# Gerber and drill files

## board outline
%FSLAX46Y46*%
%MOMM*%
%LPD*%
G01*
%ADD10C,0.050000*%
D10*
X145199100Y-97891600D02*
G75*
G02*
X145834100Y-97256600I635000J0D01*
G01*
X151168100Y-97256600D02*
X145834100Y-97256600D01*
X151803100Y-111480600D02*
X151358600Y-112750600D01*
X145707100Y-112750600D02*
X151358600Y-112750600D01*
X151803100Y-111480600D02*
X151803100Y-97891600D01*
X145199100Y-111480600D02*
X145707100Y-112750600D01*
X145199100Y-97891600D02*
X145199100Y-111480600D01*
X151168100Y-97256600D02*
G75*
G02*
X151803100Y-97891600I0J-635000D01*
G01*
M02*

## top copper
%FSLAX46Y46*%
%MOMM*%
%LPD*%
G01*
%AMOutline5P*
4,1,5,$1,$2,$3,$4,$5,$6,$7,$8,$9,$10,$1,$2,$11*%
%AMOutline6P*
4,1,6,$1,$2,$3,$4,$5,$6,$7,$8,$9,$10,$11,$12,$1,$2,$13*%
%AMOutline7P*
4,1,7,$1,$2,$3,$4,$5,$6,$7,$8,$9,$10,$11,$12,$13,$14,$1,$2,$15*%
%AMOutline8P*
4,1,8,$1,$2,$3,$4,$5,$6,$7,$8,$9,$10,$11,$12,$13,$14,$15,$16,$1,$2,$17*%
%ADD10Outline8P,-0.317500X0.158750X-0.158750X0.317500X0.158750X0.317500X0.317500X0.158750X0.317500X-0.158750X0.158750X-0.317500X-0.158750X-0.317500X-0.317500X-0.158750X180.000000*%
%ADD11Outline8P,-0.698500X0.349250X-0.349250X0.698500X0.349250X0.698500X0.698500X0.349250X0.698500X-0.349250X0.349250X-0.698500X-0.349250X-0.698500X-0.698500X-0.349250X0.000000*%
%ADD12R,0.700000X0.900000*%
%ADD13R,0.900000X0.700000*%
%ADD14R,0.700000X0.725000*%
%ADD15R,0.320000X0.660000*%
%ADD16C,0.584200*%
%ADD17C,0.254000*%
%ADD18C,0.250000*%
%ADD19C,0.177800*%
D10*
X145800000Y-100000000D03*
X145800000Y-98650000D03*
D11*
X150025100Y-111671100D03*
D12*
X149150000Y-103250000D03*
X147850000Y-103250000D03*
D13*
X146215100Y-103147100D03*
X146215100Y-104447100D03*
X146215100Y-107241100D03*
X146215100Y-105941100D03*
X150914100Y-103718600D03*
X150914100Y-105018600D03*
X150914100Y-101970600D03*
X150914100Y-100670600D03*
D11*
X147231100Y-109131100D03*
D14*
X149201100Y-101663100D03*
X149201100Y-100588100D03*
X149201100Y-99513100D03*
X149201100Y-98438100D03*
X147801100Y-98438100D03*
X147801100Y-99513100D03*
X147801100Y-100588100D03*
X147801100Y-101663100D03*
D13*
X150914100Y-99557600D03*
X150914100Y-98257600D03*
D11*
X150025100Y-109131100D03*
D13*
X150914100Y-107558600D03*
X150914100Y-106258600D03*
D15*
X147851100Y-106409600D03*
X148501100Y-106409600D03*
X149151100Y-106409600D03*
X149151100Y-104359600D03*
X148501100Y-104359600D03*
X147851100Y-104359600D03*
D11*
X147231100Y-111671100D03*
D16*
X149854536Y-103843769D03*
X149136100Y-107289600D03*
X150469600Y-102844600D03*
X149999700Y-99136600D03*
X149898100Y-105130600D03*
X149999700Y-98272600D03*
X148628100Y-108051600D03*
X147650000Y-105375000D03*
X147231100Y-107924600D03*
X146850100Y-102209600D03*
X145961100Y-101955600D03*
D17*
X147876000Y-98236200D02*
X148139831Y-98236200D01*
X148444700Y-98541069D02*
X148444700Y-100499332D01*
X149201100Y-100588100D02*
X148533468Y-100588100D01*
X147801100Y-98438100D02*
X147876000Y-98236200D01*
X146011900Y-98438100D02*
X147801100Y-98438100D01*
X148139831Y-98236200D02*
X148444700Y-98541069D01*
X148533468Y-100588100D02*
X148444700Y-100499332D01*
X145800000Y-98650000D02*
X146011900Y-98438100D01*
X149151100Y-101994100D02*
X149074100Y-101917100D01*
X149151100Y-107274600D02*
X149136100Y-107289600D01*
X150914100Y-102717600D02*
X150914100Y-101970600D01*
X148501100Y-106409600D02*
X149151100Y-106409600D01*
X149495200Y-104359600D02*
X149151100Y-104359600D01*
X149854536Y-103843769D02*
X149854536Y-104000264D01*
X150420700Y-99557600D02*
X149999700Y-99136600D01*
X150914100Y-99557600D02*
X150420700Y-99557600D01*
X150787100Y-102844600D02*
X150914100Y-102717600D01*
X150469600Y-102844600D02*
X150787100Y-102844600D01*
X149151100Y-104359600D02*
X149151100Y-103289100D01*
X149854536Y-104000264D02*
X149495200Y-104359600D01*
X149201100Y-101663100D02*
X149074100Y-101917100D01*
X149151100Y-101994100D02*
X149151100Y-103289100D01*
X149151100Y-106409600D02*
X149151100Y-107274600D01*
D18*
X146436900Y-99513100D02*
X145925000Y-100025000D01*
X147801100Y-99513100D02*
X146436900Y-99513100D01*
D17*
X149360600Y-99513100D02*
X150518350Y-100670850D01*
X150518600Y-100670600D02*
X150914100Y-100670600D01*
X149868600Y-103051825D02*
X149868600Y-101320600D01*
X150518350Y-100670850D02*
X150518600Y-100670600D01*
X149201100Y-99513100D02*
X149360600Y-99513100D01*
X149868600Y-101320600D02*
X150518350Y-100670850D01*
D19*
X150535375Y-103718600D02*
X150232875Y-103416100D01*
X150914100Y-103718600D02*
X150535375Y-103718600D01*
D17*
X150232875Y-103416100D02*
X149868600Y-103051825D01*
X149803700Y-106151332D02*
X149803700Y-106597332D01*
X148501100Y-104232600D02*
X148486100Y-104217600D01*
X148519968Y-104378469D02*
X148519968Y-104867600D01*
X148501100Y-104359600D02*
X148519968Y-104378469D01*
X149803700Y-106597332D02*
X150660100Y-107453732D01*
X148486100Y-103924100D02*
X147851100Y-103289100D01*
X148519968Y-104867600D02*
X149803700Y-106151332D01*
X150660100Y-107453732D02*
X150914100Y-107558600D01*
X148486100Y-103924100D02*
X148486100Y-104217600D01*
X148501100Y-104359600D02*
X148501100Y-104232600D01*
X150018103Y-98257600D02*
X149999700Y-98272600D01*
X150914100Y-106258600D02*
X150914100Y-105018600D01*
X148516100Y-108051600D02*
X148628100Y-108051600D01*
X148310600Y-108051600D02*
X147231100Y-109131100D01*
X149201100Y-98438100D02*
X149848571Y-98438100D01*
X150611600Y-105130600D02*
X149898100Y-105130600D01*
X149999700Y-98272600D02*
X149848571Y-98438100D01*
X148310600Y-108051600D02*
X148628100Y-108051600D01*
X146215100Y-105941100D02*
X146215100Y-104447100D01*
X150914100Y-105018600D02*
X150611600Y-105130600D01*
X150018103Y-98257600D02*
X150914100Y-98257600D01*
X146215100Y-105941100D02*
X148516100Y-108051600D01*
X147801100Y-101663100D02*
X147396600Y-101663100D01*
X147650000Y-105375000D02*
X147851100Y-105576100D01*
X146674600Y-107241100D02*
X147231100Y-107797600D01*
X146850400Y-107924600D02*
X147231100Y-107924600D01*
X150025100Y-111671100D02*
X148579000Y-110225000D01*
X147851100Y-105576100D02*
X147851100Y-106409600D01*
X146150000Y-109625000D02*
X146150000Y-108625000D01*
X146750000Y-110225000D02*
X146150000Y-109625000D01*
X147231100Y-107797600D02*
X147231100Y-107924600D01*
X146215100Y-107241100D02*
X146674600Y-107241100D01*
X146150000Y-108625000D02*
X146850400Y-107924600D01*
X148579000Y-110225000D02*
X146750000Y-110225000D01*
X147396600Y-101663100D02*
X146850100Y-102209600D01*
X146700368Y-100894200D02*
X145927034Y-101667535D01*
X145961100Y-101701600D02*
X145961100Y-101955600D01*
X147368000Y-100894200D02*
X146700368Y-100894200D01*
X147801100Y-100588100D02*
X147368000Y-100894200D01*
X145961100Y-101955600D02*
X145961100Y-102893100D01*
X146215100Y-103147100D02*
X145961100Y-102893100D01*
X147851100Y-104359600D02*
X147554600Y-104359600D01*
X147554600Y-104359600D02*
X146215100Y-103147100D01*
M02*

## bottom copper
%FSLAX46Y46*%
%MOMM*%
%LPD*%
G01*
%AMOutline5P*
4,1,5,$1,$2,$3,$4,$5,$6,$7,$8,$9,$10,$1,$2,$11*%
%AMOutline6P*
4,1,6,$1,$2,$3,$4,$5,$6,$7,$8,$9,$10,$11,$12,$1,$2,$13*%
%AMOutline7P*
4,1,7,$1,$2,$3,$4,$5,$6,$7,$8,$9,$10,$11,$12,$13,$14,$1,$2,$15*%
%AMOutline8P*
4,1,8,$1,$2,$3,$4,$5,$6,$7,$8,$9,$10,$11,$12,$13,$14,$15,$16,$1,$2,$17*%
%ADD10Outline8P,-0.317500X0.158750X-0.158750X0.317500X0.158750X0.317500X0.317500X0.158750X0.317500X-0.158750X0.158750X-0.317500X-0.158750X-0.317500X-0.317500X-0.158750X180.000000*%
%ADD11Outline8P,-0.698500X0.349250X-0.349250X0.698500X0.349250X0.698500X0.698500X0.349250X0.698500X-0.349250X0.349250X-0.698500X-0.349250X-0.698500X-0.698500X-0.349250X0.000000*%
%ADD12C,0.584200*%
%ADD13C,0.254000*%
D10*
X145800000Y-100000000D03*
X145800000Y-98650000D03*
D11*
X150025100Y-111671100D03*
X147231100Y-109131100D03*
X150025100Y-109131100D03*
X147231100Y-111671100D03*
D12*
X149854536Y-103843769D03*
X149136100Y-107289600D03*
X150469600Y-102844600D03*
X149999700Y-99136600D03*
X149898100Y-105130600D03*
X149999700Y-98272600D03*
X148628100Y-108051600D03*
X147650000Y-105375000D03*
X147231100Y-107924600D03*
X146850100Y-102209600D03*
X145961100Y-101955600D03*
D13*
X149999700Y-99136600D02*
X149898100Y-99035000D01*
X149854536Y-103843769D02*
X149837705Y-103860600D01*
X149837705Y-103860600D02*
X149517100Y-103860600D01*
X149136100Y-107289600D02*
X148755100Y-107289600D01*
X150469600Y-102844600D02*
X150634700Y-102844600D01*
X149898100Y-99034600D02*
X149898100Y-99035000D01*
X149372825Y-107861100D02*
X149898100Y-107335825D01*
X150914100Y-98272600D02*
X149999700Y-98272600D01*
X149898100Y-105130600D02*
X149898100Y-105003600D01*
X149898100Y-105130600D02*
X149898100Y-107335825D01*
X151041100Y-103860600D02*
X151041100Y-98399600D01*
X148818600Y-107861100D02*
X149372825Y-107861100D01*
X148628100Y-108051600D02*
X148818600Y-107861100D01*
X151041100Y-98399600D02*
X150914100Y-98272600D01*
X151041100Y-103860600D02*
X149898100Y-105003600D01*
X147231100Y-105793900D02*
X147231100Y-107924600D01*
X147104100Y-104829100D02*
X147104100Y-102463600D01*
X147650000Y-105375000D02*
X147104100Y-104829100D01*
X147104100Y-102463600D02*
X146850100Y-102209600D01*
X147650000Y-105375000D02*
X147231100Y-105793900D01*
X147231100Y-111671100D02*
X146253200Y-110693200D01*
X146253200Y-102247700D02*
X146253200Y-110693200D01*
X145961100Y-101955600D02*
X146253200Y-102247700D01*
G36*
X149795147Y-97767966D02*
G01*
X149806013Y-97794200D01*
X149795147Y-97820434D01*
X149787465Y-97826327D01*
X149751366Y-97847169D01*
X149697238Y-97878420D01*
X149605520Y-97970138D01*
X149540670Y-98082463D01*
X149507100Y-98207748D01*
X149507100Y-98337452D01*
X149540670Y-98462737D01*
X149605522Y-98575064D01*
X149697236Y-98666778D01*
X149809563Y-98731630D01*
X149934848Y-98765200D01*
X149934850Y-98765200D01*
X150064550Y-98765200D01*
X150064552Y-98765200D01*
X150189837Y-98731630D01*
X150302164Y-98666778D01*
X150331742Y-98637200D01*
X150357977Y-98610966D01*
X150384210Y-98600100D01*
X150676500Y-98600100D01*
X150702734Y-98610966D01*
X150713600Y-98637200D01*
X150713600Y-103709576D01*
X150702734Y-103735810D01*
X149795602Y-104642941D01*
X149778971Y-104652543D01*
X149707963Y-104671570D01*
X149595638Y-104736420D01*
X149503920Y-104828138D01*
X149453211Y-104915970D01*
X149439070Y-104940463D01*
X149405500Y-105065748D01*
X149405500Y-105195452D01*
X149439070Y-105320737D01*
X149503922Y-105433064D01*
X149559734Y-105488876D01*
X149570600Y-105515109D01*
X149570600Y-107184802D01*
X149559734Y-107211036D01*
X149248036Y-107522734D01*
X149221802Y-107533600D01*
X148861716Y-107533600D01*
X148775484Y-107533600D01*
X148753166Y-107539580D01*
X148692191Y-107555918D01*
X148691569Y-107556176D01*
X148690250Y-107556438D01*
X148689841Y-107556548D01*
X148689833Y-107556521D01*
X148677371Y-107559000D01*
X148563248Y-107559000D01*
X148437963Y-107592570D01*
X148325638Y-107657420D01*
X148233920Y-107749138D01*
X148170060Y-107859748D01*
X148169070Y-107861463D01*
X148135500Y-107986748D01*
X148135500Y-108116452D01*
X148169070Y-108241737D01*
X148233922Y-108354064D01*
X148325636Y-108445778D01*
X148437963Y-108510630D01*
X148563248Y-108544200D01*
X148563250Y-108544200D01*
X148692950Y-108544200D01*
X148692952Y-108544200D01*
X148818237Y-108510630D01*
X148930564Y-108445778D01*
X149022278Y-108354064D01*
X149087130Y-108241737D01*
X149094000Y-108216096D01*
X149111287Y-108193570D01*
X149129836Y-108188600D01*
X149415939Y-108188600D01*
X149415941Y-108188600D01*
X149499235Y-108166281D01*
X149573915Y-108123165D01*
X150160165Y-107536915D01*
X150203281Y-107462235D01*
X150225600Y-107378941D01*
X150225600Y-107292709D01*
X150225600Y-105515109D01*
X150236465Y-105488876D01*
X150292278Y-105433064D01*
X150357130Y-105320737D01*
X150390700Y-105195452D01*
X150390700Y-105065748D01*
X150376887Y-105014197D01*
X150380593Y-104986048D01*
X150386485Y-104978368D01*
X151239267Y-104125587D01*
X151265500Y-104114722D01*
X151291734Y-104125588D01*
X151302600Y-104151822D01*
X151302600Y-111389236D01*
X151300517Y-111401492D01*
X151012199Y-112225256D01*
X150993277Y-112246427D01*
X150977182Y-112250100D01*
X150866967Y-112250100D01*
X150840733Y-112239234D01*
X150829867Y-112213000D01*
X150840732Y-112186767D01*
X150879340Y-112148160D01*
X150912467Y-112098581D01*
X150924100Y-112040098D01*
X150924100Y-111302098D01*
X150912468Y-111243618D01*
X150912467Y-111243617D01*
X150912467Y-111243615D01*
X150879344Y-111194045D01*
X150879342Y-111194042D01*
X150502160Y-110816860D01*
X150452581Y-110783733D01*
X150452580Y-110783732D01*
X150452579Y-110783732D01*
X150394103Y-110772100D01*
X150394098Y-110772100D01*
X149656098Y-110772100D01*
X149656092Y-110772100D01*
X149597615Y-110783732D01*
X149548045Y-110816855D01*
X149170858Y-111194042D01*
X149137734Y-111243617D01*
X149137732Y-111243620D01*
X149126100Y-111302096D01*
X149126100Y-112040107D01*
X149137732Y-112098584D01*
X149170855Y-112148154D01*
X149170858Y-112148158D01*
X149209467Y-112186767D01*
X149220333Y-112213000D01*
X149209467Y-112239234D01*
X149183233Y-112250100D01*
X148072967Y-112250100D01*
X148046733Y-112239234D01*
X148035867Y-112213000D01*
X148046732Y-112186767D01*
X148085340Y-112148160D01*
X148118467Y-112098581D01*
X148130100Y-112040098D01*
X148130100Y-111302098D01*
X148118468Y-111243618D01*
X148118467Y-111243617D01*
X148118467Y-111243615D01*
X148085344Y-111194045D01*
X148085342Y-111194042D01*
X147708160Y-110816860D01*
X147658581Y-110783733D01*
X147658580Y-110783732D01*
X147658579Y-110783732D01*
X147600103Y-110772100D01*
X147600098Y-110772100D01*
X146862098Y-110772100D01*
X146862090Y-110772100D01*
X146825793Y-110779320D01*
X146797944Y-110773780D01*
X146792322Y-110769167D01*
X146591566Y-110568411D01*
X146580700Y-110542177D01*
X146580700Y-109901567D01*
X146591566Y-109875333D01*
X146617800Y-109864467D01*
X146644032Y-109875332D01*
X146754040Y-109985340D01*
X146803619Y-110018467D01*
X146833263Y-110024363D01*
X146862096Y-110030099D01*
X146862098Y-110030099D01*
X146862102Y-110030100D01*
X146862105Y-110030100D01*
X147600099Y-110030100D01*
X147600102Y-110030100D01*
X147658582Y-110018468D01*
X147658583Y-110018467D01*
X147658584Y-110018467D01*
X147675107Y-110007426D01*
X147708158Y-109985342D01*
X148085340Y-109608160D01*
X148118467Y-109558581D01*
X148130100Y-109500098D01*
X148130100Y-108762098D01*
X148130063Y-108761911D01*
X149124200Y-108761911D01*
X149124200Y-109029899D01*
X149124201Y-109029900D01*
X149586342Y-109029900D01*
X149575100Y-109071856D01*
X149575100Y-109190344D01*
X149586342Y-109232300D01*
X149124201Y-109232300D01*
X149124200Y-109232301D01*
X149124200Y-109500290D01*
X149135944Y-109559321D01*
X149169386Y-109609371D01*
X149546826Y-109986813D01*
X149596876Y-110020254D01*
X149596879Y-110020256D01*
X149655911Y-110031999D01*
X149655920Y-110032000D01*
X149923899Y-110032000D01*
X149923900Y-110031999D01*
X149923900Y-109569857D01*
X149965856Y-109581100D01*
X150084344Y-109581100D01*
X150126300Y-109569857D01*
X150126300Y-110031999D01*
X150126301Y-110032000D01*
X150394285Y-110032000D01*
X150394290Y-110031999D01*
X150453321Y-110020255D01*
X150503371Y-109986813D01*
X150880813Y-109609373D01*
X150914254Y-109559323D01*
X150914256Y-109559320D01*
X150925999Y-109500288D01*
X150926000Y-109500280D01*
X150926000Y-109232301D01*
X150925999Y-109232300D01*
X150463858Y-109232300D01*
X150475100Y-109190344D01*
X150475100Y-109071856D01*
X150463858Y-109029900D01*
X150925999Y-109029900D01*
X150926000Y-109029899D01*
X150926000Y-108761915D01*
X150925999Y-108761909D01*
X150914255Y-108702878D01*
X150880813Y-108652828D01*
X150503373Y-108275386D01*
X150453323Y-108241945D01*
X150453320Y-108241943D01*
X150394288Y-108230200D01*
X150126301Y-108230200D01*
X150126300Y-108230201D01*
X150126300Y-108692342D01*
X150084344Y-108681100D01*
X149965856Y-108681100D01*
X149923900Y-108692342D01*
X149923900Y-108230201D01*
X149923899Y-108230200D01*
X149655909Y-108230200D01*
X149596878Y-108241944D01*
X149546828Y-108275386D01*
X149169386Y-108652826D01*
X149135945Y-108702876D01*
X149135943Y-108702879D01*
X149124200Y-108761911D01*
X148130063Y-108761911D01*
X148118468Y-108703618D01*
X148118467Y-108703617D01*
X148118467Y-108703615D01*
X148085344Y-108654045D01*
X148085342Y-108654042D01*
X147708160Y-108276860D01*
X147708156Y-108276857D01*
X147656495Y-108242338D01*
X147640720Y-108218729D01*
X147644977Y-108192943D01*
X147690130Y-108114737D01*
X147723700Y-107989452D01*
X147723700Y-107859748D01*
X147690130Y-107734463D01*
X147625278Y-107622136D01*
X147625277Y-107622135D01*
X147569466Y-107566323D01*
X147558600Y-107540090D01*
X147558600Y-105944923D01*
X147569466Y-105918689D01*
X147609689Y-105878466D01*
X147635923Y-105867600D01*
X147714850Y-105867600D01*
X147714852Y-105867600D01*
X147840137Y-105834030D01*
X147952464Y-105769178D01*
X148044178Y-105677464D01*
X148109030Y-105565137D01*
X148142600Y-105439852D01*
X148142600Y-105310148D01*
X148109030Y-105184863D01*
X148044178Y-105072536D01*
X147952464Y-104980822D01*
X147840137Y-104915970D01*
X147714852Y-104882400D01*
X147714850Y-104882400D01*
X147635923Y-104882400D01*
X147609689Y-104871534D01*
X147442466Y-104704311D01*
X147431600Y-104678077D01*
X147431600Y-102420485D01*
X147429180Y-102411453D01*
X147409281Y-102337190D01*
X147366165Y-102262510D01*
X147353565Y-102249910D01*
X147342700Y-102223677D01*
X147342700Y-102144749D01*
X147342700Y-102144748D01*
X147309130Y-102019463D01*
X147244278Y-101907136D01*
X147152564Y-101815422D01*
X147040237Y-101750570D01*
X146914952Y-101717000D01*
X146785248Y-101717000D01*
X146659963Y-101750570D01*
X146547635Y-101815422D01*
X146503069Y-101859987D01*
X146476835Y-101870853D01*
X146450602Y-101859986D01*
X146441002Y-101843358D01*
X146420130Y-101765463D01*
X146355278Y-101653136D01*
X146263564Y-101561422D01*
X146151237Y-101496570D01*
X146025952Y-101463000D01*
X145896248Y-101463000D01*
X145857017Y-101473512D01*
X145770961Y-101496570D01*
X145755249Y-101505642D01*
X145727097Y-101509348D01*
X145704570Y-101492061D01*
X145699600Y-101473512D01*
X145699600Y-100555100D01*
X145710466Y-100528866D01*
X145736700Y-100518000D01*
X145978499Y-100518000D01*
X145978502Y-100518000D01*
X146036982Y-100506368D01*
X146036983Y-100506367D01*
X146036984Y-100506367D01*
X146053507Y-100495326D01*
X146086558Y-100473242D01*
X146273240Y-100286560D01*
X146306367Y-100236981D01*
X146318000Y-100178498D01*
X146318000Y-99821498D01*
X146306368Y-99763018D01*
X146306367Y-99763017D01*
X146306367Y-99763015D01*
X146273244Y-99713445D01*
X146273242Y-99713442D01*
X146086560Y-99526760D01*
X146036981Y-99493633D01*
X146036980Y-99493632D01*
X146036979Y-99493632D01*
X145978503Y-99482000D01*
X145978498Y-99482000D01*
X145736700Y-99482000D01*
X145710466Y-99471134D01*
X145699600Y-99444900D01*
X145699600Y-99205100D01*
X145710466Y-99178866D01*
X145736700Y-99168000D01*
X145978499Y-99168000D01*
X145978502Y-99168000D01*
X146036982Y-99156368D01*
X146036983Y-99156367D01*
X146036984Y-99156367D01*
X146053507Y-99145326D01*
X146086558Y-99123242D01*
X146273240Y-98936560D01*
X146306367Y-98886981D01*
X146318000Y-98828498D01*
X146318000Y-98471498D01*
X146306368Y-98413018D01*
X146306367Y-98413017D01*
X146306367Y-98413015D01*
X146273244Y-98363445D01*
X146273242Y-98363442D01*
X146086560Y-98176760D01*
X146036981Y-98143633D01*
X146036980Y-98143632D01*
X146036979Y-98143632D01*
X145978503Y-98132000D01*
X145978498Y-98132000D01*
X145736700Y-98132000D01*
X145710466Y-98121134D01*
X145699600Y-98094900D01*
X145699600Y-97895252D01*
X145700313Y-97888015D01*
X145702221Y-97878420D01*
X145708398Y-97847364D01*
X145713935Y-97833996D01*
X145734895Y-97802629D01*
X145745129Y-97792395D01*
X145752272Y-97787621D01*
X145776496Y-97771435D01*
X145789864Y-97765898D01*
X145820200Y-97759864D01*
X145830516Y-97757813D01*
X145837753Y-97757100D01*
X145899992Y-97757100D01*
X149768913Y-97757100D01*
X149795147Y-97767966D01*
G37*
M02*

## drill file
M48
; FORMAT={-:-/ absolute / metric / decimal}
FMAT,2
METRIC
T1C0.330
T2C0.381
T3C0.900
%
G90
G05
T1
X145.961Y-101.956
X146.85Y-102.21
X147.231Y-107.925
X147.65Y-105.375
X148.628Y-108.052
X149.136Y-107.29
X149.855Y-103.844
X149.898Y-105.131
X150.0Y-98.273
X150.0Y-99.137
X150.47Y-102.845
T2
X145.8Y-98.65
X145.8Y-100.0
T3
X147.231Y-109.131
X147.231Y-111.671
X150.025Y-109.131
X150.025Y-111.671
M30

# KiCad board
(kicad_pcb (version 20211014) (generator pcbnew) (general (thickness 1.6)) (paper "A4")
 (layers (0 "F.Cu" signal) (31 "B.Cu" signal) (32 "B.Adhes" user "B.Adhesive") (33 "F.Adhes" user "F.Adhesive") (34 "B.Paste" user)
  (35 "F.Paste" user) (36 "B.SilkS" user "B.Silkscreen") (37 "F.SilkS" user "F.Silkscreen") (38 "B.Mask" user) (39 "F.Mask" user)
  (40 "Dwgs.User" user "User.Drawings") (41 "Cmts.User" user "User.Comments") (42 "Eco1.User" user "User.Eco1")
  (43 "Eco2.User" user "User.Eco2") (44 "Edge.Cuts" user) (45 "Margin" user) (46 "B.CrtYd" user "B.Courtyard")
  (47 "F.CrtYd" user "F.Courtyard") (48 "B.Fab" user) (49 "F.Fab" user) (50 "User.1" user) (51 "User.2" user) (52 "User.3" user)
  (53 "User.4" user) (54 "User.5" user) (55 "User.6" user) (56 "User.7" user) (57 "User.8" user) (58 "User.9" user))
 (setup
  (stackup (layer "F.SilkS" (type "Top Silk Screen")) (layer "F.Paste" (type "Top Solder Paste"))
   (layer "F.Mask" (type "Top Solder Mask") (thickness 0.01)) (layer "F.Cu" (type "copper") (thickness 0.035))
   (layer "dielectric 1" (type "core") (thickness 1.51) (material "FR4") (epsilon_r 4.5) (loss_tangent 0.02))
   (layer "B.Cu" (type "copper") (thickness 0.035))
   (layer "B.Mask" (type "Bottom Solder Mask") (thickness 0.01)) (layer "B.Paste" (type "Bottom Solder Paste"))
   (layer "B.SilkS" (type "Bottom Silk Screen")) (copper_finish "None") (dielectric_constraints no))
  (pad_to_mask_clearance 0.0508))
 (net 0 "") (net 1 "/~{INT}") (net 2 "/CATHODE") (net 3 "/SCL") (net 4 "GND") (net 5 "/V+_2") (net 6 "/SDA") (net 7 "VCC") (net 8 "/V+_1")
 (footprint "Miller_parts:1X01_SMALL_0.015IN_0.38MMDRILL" (layer "F.Cu") (at 145.8 100)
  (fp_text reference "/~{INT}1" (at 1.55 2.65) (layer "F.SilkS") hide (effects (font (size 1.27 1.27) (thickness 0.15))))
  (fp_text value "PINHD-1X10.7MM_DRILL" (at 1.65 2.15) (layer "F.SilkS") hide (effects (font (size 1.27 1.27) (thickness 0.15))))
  (pad "P$1" thru_hole roundrect (at 0 0 180) (size 0.635 0.635) (drill 0.381) (layers *.Cu *.Mask) (roundrect_rratio 0.25)
   (chamfer_ratio 0.25) (chamfer top_left top_right bottom_left bottom_right) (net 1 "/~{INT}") (solder_mask_margin 0.0635)))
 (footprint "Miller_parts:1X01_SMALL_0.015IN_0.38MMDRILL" (layer "F.Cu") (at 145.8 98.65)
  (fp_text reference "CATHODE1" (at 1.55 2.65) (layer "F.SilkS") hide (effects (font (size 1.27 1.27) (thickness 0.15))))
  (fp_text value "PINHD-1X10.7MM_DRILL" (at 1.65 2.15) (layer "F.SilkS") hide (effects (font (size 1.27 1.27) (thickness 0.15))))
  (pad "P$1" thru_hole roundrect (at 0 0 180) (size 0.635 0.635) (drill 0.381) (layers *.Cu *.Mask) (roundrect_rratio 0.25)
   (chamfer_ratio 0.25) (chamfer top_left top_right bottom_left bottom_right) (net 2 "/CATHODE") (solder_mask_margin 0.0635)))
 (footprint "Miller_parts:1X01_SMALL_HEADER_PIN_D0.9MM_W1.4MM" (layer "F.Cu") (at 150.0251 111.6711)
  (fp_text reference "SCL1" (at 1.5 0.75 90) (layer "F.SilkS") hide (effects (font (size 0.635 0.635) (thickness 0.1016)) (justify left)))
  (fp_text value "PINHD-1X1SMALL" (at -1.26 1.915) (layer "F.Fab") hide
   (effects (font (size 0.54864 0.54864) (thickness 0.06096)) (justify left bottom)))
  (pad "1" thru_hole roundrect (at 0 0) (size 1.397 1.397) (drill 0.9) (layers *.Cu *.Mask) (roundrect_rratio 0.25) (chamfer_ratio 0.25)
   (chamfer top_left top_right bottom_left bottom_right) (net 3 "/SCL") (solder_mask_margin 0.0635)))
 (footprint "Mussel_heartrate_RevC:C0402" (layer "F.Cu") (at 148.5 103.25 180)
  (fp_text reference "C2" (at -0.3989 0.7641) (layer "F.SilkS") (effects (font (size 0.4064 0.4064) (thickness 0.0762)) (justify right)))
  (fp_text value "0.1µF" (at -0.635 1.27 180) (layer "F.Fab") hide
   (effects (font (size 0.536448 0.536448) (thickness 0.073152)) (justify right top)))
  (pad "1" smd rect (at -0.65 0 180) (size 0.7 0.9) (layers "F.Cu" "F.Paste" "F.Mask") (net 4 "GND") (solder_mask_margin 0.0635))
  (pad "2" smd rect (at 0.65 0 180) (size 0.7 0.9) (layers "F.Cu" "F.Paste" "F.Mask") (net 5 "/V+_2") (solder_mask_margin 0.0635)))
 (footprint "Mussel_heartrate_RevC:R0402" (layer "F.Cu") (at 146.2151 103.7971 -90)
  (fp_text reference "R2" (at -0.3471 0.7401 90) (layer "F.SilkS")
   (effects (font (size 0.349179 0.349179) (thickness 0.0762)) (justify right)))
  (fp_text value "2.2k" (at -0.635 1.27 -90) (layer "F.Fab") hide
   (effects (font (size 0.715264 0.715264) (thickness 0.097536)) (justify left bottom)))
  (pad "1" smd rect (at -0.65 0 270) (size 0.7 0.9) (layers "F.Cu" "F.Paste" "F.Mask") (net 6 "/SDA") (solder_mask_margin 0.0635))
  (pad "2" smd rect (at 0.65 0 270) (size 0.7 0.9) (layers "F.Cu" "F.Paste" "F.Mask") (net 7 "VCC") (solder_mask_margin 0.0635)))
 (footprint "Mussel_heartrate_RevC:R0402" (layer "F.Cu") (at 146.2151 106.5911 90)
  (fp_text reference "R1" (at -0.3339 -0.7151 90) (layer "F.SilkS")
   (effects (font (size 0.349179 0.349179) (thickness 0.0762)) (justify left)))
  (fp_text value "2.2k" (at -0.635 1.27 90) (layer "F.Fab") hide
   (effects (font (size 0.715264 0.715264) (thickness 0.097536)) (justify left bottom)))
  (pad "1" smd rect (at -0.65 0 90) (size 0.7 0.9) (layers "F.Cu" "F.Paste" "F.Mask") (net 3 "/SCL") (solder_mask_margin 0.0635))
  (pad "2" smd rect (at 0.65 0 90) (size 0.7 0.9) (layers "F.Cu" "F.Paste" "F.Mask") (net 7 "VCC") (solder_mask_margin 0.0635)))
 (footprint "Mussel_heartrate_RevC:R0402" (layer "F.Cu") (at 150.9141 104.3686 -90)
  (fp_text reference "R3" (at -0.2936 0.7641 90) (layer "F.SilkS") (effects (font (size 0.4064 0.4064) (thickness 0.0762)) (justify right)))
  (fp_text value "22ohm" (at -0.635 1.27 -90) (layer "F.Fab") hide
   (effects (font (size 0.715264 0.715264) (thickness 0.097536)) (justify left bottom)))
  (pad "1" smd rect (at -0.65 0 270) (size 0.7 0.9) (layers "F.Cu" "F.Paste" "F.Mask") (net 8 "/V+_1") (solder_mask_margin 0.0635))
  (pad "2" smd rect (at 0.65 0 270) (size 0.7 0.9) (layers "F.Cu" "F.Paste" "F.Mask") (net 7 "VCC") (solder_mask_margin 0.0635)))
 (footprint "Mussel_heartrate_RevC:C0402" (layer "F.Cu") (at 150.9141 101.3206 90)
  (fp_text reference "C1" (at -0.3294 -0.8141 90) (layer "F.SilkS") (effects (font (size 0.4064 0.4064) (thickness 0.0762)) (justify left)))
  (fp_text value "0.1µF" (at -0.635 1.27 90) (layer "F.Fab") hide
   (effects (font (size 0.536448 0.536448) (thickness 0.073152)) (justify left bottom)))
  (pad "1" smd rect (at -0.65 0 90) (size 0.7 0.9) (layers "F.Cu" "F.Paste" "F.Mask") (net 4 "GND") (solder_mask_margin 0.0635))
  (pad "2" smd rect (at 0.65 0 90) (size 0.7 0.9) (layers "F.Cu" "F.Paste" "F.Mask") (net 8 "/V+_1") (solder_mask_margin 0.0635)))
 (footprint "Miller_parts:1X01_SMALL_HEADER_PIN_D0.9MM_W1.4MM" (layer "F.Cu") (at 147.2311 109.1311)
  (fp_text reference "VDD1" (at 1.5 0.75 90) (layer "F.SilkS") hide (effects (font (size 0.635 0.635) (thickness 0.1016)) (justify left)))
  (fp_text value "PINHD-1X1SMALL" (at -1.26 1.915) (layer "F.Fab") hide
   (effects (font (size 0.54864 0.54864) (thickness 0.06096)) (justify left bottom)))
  (pad "1" thru_hole roundrect (at 0 0) (size 1.397 1.397) (drill 0.9) (layers *.Cu *.Mask) (roundrect_rratio 0.25) (chamfer_ratio 0.25)
   (chamfer top_left top_right bottom_left bottom_right) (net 7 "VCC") (solder_mask_margin 0.0635)))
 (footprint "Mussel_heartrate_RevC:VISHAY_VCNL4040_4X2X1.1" (layer "F.Cu") (at 148.5011 100.0506 180)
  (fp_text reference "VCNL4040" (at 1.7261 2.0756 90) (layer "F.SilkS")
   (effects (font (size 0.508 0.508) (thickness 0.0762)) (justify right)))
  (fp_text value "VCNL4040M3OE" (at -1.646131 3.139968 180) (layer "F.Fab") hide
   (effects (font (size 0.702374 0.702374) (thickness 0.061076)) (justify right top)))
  (pad "1" smd rect (at -0.7 -1.6125 180) (size 0.7 0.725) (layers "F.Cu" "F.Paste" "F.Mask") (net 4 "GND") (solder_mask_margin 0.0635))
  (pad "2" smd rect (at -0.7 -0.5375 180) (size 0.7 0.725) (layers "F.Cu" "F.Paste" "F.Mask") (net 2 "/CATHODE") (solder_mask_margin 0.0635))
  (pad "3" smd rect (at -0.7 0.5375 180) (size 0.7 0.725) (layers "F.Cu" "F.Paste" "F.Mask") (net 8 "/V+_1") (solder_mask_margin 0.0635))
  (pad "4" smd rect (at -0.7 1.6125 180) (size 0.7 0.725) (layers "F.Cu" "F.Paste" "F.Mask") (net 7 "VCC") (solder_mask_margin 0.0635))
  (pad "5" smd rect (at 0.7 1.6125 180) (size 0.7 0.725) (layers "F.Cu" "F.Paste" "F.Mask") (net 2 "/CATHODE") (solder_mask_margin 0.0635))
  (pad "6" smd rect (at 0.7 0.5375 180) (size 0.7 0.725) (layers "F.Cu" "F.Paste" "F.Mask") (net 1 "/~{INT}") (solder_mask_margin 0.0635))
  (pad "7" smd rect (at 0.7 -0.5375 180) (size 0.7 0.725) (layers "F.Cu" "F.Paste" "F.Mask") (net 6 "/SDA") (solder_mask_margin 0.0635))
  (pad "8" smd rect (at 0.7 -1.6125 180) (size 0.7 0.725) (layers "F.Cu" "F.Paste" "F.Mask") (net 3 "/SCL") (solder_mask_margin 0.0635)))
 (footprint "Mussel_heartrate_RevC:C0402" (layer "F.Cu") (at 150.9141 98.9076 90)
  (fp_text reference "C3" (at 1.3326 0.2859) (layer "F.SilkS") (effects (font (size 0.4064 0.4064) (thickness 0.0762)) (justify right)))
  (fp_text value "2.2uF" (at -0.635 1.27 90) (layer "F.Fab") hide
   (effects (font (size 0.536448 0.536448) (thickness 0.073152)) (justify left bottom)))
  (pad "1" smd rect (at -0.65 0 90) (size 0.7 0.9) (layers "F.Cu" "F.Paste" "F.Mask") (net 4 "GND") (solder_mask_margin 0.0635))
  (pad "2" smd rect (at 0.65 0 90) (size 0.7 0.9) (layers "F.Cu" "F.Paste" "F.Mask") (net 7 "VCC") (solder_mask_margin 0.0635)))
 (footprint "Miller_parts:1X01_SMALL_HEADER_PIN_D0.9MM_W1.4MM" (layer "F.Cu") (at 150.0251 109.1311)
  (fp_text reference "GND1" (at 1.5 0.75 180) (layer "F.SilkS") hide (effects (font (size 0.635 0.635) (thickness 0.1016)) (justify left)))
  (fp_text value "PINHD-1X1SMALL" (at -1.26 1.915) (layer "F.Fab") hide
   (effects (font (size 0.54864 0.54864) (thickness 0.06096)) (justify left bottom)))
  (pad "1" thru_hole roundrect (at 0 0) (size 1.397 1.397) (drill 0.9) (layers *.Cu *.Mask) (roundrect_rratio 0.25) (chamfer_ratio 0.25)
   (chamfer top_left top_right bottom_left bottom_right) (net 4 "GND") (solder_mask_margin 0.0635)))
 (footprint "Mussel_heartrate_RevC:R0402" (layer "F.Cu") (at 150.9141 106.9086 90)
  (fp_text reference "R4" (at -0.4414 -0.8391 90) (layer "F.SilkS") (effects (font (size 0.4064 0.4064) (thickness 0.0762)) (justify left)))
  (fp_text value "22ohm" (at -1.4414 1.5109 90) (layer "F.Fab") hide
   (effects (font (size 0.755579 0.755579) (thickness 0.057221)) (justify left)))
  (pad "1" smd rect (at -0.65 0 90) (size 0.7 0.9) (layers "F.Cu" "F.Paste" "F.Mask") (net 5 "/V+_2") (solder_mask_margin 0.0635))
  (pad "2" smd rect (at 0.65 0 90) (size 0.7 0.9) (layers "F.Cu" "F.Paste" "F.Mask") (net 7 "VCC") (solder_mask_margin 0.0635)))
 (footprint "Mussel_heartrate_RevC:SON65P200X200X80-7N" (layer "F.Cu") (at 148.5011 105.3846 90)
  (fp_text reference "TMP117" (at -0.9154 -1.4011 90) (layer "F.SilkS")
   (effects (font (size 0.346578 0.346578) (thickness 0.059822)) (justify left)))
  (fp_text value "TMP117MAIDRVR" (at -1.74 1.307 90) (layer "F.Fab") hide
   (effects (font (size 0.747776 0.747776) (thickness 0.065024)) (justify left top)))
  (pad "1" smd rect (at -1.025 -0.65 90) (size 0.66 0.32) (layers "F.Cu" "F.Paste" "F.Mask") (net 3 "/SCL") (solder_mask_margin 0.0635))
  (pad "2" smd rect (at -1.025 0 90) (size 0.66 0.32) (layers "F.Cu" "F.Paste" "F.Mask") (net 4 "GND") (solder_mask_margin 0.0635))
  (pad "3" smd rect (at -1.025 0.65 90) (size 0.66 0.32) (layers "F.Cu" "F.Paste" "F.Mask") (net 4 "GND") (solder_mask_margin 0.0635))
  (pad "4" smd rect (at 1.025 0.65 90) (size 0.66 0.32) (layers "F.Cu" "F.Paste" "F.Mask") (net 4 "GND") (solder_mask_margin 0.0635))
  (pad "5" smd rect (at 1.025 0 90) (size 0.66 0.32) (layers "F.Cu" "F.Paste" "F.Mask") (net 5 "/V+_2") (solder_mask_margin 0.0635))
  (pad "6" smd rect (at 1.025 -0.65 90) (size 0.66 0.32) (layers "F.Cu" "F.Paste" "F.Mask") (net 6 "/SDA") (solder_mask_margin 0.0635)))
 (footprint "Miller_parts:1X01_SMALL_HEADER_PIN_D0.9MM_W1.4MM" (layer "F.Cu") (at 147.2311 111.6711)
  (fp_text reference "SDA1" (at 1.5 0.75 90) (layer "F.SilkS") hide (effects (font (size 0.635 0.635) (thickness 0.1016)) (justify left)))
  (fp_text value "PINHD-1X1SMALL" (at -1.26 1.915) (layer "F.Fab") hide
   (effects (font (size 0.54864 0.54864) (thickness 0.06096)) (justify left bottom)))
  (pad "1" thru_hole roundrect (at 0 0) (size 1.397 1.397) (drill 0.9) (layers *.Cu *.Mask) (roundrect_rratio 0.25) (chamfer_ratio 0.25)
   (chamfer top_left top_right bottom_left bottom_right) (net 6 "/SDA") (solder_mask_margin 0.0635)))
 (gr_arc (start 145.1991 97.8916) (mid 145.385087 97.442587) (end 145.8341 97.2566) (layer "Edge.Cuts") (width 0.05))
 (gr_line (start 151.1681 97.2566) (end 145.8341 97.2566) (layer "Edge.Cuts") (width 0.05))
 (gr_line (start 151.8031 111.4806) (end 151.3586 112.7506) (layer "Edge.Cuts") (width 0.05))
 (gr_line (start 145.7071 112.7506) (end 151.3586 112.7506) (layer "Edge.Cuts") (width 0.05))
 (gr_line (start 151.8031 111.4806) (end 151.8031 97.8916) (layer "Edge.Cuts") (width 0.05))
 (gr_line (start 145.1991 111.4806) (end 145.7071 112.7506) (layer "Edge.Cuts") (width 0.05))
 (gr_line (start 145.1991 97.8916) (end 145.1991 111.4806) (layer "Edge.Cuts") (width 0.05))
 (gr_arc (start 151.1681 97.2566) (mid 151.617113 97.442587) (end 151.8031 97.8916) (layer "Edge.Cuts") (width 0.05))
 (segment (start 147.876 98.2362) (end 148.139831 98.2362) (width 0.254) (layer "F.Cu") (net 2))
 (segment (start 148.4447 98.541069) (end 148.4447 100.499332) (width 0.254) (layer "F.Cu") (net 2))
 (segment (start 149.2011 100.5881) (end 148.533468 100.5881) (width 0.254) (layer "F.Cu") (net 2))
 (segment (start 147.8011 98.4381) (end 147.876 98.2362) (width 0.254) (layer "F.Cu") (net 2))
 (segment (start 146.0119 98.4381) (end 147.8011 98.4381) (width 0.254) (layer "F.Cu") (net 2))
 (segment (start 148.139831 98.2362) (end 148.4447 98.541069) (width 0.254) (layer "F.Cu") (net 2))
 (segment (start 148.533468 100.5881) (end 148.4447 100.499332) (width 0.254) (layer "F.Cu") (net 2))
 (segment (start 145.8 98.65) (end 146.0119 98.4381) (width 0.254) (layer "F.Cu") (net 2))
 (segment (start 149.1511 101.9941) (end 149.0741 101.9171) (width 0.254) (layer "F.Cu") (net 4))
 (segment (start 149.1511 107.2746) (end 149.1361 107.2896) (width 0.254) (layer "F.Cu") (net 4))
 (segment (start 150.9141 102.7176) (end 150.9141 101.9706) (width 0.254) (layer "F.Cu") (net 4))
 (segment (start 148.5011 106.4096) (end 149.1511 106.4096) (width 0.254) (layer "F.Cu") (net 4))
 (segment (start 149.4952 104.3596) (end 149.1511 104.3596) (width 0.254) (layer "F.Cu") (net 4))
 (segment (start 149.854536 103.843769) (end 149.854536 104.000264) (width 0.254) (layer "F.Cu") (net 4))
 (segment (start 150.4207 99.5576) (end 149.9997 99.1366) (width 0.254) (layer "F.Cu") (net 4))
 (segment (start 150.9141 99.5576) (end 150.4207 99.5576) (width 0.254) (layer "F.Cu") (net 4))
 (segment (start 150.7871 102.8446) (end 150.9141 102.7176) (width 0.254) (layer "F.Cu") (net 4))
 (segment (start 150.4696 102.8446) (end 150.7871 102.8446) (width 0.254) (layer "F.Cu") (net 4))
 (segment (start 149.1511 104.3596) (end 149.1511 103.2891) (width 0.254) (layer "F.Cu") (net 4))
 (segment (start 149.854536 104.000264) (end 149.4952 104.3596) (width 0.254) (layer "F.Cu") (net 4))
 (segment (start 149.2011 101.6631) (end 149.0741 101.9171) (width 0.254) (layer "F.Cu") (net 4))
 (segment (start 149.1511 101.9941) (end 149.1511 103.2891) (width 0.254) (layer "F.Cu") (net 4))
 (segment (start 149.1511 106.4096) (end 149.1511 107.2746) (width 0.254) (layer "F.Cu") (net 4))
 (via (at 149.854536 103.843769) (size 0.5842) (drill 0.3302) (layers "F.Cu" "B.Cu") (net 4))
 (via (at 149.1361 107.2896) (size 0.5842) (drill 0.3302) (layers "F.Cu" "B.Cu") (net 4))
 (via (at 150.4696 102.8446) (size 0.5842) (drill 0.3302) (layers "F.Cu" "B.Cu") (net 4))
 (via (at 149.9997 99.1366) (size 0.5842) (drill 0.3302) (layers "F.Cu" "B.Cu") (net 4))
 (segment (start 149.9997 99.1366) (end 149.8981 99.035) (width 0.254) (layer "B.Cu") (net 4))
 (segment (start 149.854536 103.843769) (end 149.837705 103.8606) (width 0.254) (layer "B.Cu") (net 4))
 (segment (start 149.837705 103.8606) (end 149.5171 103.8606) (width 0.254) (layer "B.Cu") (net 4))
 (segment (start 149.1361 107.2896) (end 148.7551 107.2896) (width 0.254) (layer "B.Cu") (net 4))
 (segment (start 150.4696 102.8446) (end 150.6347 102.8446) (width 0.254) (layer "B.Cu") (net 4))
 (segment (start 149.8981 99.0346) (end 149.8981 99.035) (width 0.254) (layer "B.Cu") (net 4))
 (segment (start 146.4369 99.5131) (end 145.925 100.025) (width 0.25) (layer "F.Cu") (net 1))
 (segment (start 147.8011 99.5131) (end 146.4369 99.5131) (width 0.25) (layer "F.Cu") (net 1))
 (segment (start 149.3606 99.5131) (end 150.51835 100.67085) (width 0.254) (layer "F.Cu") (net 8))
 (segment (start 150.5186 100.6706) (end 150.9141 100.6706) (width 0.254) (layer "F.Cu") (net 8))
 (segment (start 149.8686 103.051825) (end 149.8686 101.3206) (width 0.254) (layer "F.Cu") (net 8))
 (segment (start 150.51835 100.67085) (end 150.5186 100.6706) (width 0.254) (layer "F.Cu") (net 8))
 (segment (start 149.2011 99.5131) (end 149.3606 99.5131) (width 0.254) (layer "F.Cu") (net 8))
 (segment (start 149.8686 101.3206) (end 150.51835 100.67085) (width 0.254) (layer "F.Cu") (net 8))
 (segment (start 150.535375 103.7186) (end 150.232875 103.4161) (width 0.1778) (layer "F.Cu") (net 8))
 (segment (start 150.9141 103.7186) (end 150.535375 103.7186) (width 0.1778) (layer "F.Cu") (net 8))
 (segment (start 150.232875 103.4161) (end 149.8686 103.051825) (width 0.254) (layer "F.Cu") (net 8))
 (segment (start 149.8037 106.151332) (end 149.8037 106.597332) (width 0.254) (layer "F.Cu") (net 5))
 (segment (start 148.5011 104.2326) (end 148.4861 104.2176) (width 0.254) (layer "F.Cu") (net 5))
 (segment (start 148.519968 104.378469) (end 148.519968 104.8676) (width 0.254) (layer "F.Cu") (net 5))
 (segment (start 148.5011 104.3596) (end 148.519968 104.378469) (width 0.254) (layer "F.Cu") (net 5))
 (segment (start 149.8037 106.597332) (end 150.6601 107.453732) (width 0.254) (layer "F.Cu") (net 5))
 (segment (start 148.4861 103.9241) (end 147.8511 103.2891) (width 0.254) (layer "F.Cu") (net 5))
 (segment (start 148.519968 104.8676) (end 149.8037 106.151332) (width 0.254) (layer "F.Cu") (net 5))
 (segment (start 150.6601 107.453732) (end 150.9141 107.5586) (width 0.254) (layer "F.Cu") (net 5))
 (segment (start 148.4861 103.9241) (end 148.4861 104.2176) (width 0.254) (layer "F.Cu") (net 5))
 (segment (start 148.5011 104.3596) (end 148.5011 104.2326) (width 0.254) (layer "F.Cu") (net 5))
 (segment (start 150.018103 98.2576) (end 149.9997 98.2726) (width 0.254) (layer "F.Cu") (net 7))
 (segment (start 150.9141 106.2586) (end 150.9141 105.0186) (width 0.254) (layer "F.Cu") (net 7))
 (segment (start 148.5161 108.0516) (end 148.6281 108.0516) (width 0.254) (layer "F.Cu") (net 7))
 (segment (start 148.3106 108.0516) (end 147.2311 109.1311) (width 0.254) (layer "F.Cu") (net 7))
 (segment (start 149.2011 98.4381) (end 149.848571 98.4381) (width 0.254) (layer "F.Cu") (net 7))
 (segment (start 150.6116 105.1306) (end 149.8981 105.1306) (width 0.254) (layer "F.Cu") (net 7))
 (segment (start 149.9997 98.2726) (end 149.848571 98.4381) (width 0.254) (layer "F.Cu") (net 7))
 (segment (start 148.3106 108.0516) (end 148.6281 108.0516) (width 0.254) (layer "F.Cu") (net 7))
 (segment (start 146.2151 105.9411) (end 146.2151 104.4471) (width 0.254) (layer "F.Cu") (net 7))
 (segment (start 150.9141 105.0186) (end 150.6116 105.1306) (width 0.254) (layer "F.Cu") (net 7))
 (segment (start 150.018103 98.2576) (end 150.9141 98.2576) (width 0.254) (layer "F.Cu") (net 7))
 (segment (start 146.2151 105.9411) (end 148.5161 108.0516) (width 0.254) (layer "F.Cu") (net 7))
 (via (at 149.8981 105.1306) (size 0.5842) (drill 0.3302) (layers "F.Cu" "B.Cu") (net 7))
 (via (at 149.9997 98.2726) (size 0.5842) (drill 0.3302) (layers "F.Cu" "B.Cu") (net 7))
 (via (at 148.6281 108.0516) (size 0.5842) (drill 0.3302) (layers "F.Cu" "B.Cu") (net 7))
 (segment (start 149.372825 107.8611) (end 149.8981 107.335825) (width 0.254) (layer "B.Cu") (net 7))
 (segment (start 150.9141 98.2726) (end 149.9997 98.2726) (width 0.254) (layer "B.Cu") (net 7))
 (segment (start 149.8981 105.1306) (end 149.8981 105.0036) (width 0.254) (layer "B.Cu") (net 7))
 (segment (start 149.8981 105.1306) (end 149.8981 107.335825) (width 0.254) (layer "B.Cu") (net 7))
 (segment (start 151.0411 103.8606) (end 151.0411 98.3996) (width 0.254) (layer "B.Cu") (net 7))
 (segment (start 148.8186 107.8611) (end 149.372825 107.8611) (width 0.254) (layer "B.Cu") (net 7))
 (segment (start 148.6281 108.0516) (end 148.8186 107.8611) (width 0.254) (layer "B.Cu") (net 7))
 (segment (start 151.0411 98.3996) (end 150.9141 98.2726) (width 0.254) (layer "B.Cu") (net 7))
 (segment (start 151.0411 103.8606) (end 149.8981 105.0036) (width 0.254) (layer "B.Cu") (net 7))
 (segment (start 147.8011 101.6631) (end 147.3966 101.6631) (width 0.254) (layer "F.Cu") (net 3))
 (segment (start 147.65 105.375) (end 147.8511 105.5761) (width 0.254) (layer "F.Cu") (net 3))
 (segment (start 146.6746 107.2411) (end 147.2311 107.7976) (width 0.254) (layer "F.Cu") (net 3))
 (segment (start 146.8504 107.9246) (end 147.2311 107.9246) (width 0.254) (layer "F.Cu") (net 3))
 (segment (start 150.0251 111.6711) (end 148.579 110.225) (width 0.254) (layer "F.Cu") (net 3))
 (segment (start 147.8511 105.5761) (end 147.8511 106.4096) (width 0.254) (layer "F.Cu") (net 3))
 (segment (start 146.15 109.625) (end 146.15 108.625) (width 0.254) (layer "F.Cu") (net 3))
 (segment (start 146.75 110.225) (end 146.15 109.625) (width 0.254) (layer "F.Cu") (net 3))
 (segment (start 147.2311 107.7976) (end 147.2311 107.9246) (width 0.254) (layer "F.Cu") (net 3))
 (segment (start 146.2151 107.2411) (end 146.6746 107.2411) (width 0.254) (layer "F.Cu") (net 3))
 (segment (start 146.15 108.625) (end 146.8504 107.9246) (width 0.254) (layer "F.Cu") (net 3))
 (segment (start 148.579 110.225) (end 146.75 110.225) (width 0.254) (layer "F.Cu") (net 3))
 (segment (start 147.3966 101.6631) (end 146.8501 102.2096) (width 0.254) (layer "F.Cu") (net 3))
 (via (at 147.65 105.375) (size 0.5842) (drill 0.3302) (layers "F.Cu" "B.Cu") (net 3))
 (via (at 147.2311 107.9246) (size 0.5842) (drill 0.3302) (layers "F.Cu" "B.Cu") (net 3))
 (via (at 146.8501 102.2096) (size 0.5842) (drill 0.3302) (layers "F.Cu" "B.Cu") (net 3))
 (segment (start 147.2311 105.7939) (end 147.2311 107.9246) (width 0.254) (layer "B.Cu") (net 3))
 (segment (start 147.1041 104.8291) (end 147.1041 102.4636) (width 0.254) (layer "B.Cu") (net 3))
 (segment (start 147.65 105.375) (end 147.1041 104.8291) (width 0.254) (layer "B.Cu") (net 3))
 (segment (start 147.1041 102.4636) (end 146.8501 102.2096) (width 0.254) (layer "B.Cu") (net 3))
 (segment (start 147.65 105.375) (end 147.2311 105.7939) (width 0.254) (layer "B.Cu") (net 3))
 (segment (start 146.700368 100.8942) (end 145.927034 101.667535) (width 0.254) (layer "F.Cu") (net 6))
 (segment (start 145.9611 101.7016) (end 145.9611 101.9556) (width 0.254) (layer "F.Cu") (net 6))
 (segment (start 147.368 100.8942) (end 146.700368 100.8942) (width 0.254) (layer "F.Cu") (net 6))
 (segment (start 147.8011 100.5881) (end 147.368 100.8942) (width 0.254) (layer "F.Cu") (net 6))
 (segment (start 145.9611 101.9556) (end 145.9611 102.8931) (width 0.254) (layer "F.Cu") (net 6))
 (segment (start 146.2151 103.1471) (end 145.9611 102.8931) (width 0.254) (layer "F.Cu") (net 6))
 (segment (start 147.8511 104.3596) (end 147.5546 104.3596) (width 0.254) (layer "F.Cu") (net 6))
 (segment (start 147.5546 104.3596) (end 146.2151 103.1471) (width 0.254) (layer "F.Cu") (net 6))
 (via (at 145.9611 101.9556) (size 0.5842) (drill 0.3302) (layers "F.Cu" "B.Cu") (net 6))
 (segment (start 147.2311 111.6711) (end 146.2532 110.6932) (width 0.254) (layer "B.Cu") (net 6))
 (segment (start 146.2532 102.2477) (end 146.2532 110.6932) (width 0.254) (layer "B.Cu") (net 6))
 (segment (start 145.9611 101.9556) (end 146.2532 102.2477) (width 0.254) (layer "B.Cu") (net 6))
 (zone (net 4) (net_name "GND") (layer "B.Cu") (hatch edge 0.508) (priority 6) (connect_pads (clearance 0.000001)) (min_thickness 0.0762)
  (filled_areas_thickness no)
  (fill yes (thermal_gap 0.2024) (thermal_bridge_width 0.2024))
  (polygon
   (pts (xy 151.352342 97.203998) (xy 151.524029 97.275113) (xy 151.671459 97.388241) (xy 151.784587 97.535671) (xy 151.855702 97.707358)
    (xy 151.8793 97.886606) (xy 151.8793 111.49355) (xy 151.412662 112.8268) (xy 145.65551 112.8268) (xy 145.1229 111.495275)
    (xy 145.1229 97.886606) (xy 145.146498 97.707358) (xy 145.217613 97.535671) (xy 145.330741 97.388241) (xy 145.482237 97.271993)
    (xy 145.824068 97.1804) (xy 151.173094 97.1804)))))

